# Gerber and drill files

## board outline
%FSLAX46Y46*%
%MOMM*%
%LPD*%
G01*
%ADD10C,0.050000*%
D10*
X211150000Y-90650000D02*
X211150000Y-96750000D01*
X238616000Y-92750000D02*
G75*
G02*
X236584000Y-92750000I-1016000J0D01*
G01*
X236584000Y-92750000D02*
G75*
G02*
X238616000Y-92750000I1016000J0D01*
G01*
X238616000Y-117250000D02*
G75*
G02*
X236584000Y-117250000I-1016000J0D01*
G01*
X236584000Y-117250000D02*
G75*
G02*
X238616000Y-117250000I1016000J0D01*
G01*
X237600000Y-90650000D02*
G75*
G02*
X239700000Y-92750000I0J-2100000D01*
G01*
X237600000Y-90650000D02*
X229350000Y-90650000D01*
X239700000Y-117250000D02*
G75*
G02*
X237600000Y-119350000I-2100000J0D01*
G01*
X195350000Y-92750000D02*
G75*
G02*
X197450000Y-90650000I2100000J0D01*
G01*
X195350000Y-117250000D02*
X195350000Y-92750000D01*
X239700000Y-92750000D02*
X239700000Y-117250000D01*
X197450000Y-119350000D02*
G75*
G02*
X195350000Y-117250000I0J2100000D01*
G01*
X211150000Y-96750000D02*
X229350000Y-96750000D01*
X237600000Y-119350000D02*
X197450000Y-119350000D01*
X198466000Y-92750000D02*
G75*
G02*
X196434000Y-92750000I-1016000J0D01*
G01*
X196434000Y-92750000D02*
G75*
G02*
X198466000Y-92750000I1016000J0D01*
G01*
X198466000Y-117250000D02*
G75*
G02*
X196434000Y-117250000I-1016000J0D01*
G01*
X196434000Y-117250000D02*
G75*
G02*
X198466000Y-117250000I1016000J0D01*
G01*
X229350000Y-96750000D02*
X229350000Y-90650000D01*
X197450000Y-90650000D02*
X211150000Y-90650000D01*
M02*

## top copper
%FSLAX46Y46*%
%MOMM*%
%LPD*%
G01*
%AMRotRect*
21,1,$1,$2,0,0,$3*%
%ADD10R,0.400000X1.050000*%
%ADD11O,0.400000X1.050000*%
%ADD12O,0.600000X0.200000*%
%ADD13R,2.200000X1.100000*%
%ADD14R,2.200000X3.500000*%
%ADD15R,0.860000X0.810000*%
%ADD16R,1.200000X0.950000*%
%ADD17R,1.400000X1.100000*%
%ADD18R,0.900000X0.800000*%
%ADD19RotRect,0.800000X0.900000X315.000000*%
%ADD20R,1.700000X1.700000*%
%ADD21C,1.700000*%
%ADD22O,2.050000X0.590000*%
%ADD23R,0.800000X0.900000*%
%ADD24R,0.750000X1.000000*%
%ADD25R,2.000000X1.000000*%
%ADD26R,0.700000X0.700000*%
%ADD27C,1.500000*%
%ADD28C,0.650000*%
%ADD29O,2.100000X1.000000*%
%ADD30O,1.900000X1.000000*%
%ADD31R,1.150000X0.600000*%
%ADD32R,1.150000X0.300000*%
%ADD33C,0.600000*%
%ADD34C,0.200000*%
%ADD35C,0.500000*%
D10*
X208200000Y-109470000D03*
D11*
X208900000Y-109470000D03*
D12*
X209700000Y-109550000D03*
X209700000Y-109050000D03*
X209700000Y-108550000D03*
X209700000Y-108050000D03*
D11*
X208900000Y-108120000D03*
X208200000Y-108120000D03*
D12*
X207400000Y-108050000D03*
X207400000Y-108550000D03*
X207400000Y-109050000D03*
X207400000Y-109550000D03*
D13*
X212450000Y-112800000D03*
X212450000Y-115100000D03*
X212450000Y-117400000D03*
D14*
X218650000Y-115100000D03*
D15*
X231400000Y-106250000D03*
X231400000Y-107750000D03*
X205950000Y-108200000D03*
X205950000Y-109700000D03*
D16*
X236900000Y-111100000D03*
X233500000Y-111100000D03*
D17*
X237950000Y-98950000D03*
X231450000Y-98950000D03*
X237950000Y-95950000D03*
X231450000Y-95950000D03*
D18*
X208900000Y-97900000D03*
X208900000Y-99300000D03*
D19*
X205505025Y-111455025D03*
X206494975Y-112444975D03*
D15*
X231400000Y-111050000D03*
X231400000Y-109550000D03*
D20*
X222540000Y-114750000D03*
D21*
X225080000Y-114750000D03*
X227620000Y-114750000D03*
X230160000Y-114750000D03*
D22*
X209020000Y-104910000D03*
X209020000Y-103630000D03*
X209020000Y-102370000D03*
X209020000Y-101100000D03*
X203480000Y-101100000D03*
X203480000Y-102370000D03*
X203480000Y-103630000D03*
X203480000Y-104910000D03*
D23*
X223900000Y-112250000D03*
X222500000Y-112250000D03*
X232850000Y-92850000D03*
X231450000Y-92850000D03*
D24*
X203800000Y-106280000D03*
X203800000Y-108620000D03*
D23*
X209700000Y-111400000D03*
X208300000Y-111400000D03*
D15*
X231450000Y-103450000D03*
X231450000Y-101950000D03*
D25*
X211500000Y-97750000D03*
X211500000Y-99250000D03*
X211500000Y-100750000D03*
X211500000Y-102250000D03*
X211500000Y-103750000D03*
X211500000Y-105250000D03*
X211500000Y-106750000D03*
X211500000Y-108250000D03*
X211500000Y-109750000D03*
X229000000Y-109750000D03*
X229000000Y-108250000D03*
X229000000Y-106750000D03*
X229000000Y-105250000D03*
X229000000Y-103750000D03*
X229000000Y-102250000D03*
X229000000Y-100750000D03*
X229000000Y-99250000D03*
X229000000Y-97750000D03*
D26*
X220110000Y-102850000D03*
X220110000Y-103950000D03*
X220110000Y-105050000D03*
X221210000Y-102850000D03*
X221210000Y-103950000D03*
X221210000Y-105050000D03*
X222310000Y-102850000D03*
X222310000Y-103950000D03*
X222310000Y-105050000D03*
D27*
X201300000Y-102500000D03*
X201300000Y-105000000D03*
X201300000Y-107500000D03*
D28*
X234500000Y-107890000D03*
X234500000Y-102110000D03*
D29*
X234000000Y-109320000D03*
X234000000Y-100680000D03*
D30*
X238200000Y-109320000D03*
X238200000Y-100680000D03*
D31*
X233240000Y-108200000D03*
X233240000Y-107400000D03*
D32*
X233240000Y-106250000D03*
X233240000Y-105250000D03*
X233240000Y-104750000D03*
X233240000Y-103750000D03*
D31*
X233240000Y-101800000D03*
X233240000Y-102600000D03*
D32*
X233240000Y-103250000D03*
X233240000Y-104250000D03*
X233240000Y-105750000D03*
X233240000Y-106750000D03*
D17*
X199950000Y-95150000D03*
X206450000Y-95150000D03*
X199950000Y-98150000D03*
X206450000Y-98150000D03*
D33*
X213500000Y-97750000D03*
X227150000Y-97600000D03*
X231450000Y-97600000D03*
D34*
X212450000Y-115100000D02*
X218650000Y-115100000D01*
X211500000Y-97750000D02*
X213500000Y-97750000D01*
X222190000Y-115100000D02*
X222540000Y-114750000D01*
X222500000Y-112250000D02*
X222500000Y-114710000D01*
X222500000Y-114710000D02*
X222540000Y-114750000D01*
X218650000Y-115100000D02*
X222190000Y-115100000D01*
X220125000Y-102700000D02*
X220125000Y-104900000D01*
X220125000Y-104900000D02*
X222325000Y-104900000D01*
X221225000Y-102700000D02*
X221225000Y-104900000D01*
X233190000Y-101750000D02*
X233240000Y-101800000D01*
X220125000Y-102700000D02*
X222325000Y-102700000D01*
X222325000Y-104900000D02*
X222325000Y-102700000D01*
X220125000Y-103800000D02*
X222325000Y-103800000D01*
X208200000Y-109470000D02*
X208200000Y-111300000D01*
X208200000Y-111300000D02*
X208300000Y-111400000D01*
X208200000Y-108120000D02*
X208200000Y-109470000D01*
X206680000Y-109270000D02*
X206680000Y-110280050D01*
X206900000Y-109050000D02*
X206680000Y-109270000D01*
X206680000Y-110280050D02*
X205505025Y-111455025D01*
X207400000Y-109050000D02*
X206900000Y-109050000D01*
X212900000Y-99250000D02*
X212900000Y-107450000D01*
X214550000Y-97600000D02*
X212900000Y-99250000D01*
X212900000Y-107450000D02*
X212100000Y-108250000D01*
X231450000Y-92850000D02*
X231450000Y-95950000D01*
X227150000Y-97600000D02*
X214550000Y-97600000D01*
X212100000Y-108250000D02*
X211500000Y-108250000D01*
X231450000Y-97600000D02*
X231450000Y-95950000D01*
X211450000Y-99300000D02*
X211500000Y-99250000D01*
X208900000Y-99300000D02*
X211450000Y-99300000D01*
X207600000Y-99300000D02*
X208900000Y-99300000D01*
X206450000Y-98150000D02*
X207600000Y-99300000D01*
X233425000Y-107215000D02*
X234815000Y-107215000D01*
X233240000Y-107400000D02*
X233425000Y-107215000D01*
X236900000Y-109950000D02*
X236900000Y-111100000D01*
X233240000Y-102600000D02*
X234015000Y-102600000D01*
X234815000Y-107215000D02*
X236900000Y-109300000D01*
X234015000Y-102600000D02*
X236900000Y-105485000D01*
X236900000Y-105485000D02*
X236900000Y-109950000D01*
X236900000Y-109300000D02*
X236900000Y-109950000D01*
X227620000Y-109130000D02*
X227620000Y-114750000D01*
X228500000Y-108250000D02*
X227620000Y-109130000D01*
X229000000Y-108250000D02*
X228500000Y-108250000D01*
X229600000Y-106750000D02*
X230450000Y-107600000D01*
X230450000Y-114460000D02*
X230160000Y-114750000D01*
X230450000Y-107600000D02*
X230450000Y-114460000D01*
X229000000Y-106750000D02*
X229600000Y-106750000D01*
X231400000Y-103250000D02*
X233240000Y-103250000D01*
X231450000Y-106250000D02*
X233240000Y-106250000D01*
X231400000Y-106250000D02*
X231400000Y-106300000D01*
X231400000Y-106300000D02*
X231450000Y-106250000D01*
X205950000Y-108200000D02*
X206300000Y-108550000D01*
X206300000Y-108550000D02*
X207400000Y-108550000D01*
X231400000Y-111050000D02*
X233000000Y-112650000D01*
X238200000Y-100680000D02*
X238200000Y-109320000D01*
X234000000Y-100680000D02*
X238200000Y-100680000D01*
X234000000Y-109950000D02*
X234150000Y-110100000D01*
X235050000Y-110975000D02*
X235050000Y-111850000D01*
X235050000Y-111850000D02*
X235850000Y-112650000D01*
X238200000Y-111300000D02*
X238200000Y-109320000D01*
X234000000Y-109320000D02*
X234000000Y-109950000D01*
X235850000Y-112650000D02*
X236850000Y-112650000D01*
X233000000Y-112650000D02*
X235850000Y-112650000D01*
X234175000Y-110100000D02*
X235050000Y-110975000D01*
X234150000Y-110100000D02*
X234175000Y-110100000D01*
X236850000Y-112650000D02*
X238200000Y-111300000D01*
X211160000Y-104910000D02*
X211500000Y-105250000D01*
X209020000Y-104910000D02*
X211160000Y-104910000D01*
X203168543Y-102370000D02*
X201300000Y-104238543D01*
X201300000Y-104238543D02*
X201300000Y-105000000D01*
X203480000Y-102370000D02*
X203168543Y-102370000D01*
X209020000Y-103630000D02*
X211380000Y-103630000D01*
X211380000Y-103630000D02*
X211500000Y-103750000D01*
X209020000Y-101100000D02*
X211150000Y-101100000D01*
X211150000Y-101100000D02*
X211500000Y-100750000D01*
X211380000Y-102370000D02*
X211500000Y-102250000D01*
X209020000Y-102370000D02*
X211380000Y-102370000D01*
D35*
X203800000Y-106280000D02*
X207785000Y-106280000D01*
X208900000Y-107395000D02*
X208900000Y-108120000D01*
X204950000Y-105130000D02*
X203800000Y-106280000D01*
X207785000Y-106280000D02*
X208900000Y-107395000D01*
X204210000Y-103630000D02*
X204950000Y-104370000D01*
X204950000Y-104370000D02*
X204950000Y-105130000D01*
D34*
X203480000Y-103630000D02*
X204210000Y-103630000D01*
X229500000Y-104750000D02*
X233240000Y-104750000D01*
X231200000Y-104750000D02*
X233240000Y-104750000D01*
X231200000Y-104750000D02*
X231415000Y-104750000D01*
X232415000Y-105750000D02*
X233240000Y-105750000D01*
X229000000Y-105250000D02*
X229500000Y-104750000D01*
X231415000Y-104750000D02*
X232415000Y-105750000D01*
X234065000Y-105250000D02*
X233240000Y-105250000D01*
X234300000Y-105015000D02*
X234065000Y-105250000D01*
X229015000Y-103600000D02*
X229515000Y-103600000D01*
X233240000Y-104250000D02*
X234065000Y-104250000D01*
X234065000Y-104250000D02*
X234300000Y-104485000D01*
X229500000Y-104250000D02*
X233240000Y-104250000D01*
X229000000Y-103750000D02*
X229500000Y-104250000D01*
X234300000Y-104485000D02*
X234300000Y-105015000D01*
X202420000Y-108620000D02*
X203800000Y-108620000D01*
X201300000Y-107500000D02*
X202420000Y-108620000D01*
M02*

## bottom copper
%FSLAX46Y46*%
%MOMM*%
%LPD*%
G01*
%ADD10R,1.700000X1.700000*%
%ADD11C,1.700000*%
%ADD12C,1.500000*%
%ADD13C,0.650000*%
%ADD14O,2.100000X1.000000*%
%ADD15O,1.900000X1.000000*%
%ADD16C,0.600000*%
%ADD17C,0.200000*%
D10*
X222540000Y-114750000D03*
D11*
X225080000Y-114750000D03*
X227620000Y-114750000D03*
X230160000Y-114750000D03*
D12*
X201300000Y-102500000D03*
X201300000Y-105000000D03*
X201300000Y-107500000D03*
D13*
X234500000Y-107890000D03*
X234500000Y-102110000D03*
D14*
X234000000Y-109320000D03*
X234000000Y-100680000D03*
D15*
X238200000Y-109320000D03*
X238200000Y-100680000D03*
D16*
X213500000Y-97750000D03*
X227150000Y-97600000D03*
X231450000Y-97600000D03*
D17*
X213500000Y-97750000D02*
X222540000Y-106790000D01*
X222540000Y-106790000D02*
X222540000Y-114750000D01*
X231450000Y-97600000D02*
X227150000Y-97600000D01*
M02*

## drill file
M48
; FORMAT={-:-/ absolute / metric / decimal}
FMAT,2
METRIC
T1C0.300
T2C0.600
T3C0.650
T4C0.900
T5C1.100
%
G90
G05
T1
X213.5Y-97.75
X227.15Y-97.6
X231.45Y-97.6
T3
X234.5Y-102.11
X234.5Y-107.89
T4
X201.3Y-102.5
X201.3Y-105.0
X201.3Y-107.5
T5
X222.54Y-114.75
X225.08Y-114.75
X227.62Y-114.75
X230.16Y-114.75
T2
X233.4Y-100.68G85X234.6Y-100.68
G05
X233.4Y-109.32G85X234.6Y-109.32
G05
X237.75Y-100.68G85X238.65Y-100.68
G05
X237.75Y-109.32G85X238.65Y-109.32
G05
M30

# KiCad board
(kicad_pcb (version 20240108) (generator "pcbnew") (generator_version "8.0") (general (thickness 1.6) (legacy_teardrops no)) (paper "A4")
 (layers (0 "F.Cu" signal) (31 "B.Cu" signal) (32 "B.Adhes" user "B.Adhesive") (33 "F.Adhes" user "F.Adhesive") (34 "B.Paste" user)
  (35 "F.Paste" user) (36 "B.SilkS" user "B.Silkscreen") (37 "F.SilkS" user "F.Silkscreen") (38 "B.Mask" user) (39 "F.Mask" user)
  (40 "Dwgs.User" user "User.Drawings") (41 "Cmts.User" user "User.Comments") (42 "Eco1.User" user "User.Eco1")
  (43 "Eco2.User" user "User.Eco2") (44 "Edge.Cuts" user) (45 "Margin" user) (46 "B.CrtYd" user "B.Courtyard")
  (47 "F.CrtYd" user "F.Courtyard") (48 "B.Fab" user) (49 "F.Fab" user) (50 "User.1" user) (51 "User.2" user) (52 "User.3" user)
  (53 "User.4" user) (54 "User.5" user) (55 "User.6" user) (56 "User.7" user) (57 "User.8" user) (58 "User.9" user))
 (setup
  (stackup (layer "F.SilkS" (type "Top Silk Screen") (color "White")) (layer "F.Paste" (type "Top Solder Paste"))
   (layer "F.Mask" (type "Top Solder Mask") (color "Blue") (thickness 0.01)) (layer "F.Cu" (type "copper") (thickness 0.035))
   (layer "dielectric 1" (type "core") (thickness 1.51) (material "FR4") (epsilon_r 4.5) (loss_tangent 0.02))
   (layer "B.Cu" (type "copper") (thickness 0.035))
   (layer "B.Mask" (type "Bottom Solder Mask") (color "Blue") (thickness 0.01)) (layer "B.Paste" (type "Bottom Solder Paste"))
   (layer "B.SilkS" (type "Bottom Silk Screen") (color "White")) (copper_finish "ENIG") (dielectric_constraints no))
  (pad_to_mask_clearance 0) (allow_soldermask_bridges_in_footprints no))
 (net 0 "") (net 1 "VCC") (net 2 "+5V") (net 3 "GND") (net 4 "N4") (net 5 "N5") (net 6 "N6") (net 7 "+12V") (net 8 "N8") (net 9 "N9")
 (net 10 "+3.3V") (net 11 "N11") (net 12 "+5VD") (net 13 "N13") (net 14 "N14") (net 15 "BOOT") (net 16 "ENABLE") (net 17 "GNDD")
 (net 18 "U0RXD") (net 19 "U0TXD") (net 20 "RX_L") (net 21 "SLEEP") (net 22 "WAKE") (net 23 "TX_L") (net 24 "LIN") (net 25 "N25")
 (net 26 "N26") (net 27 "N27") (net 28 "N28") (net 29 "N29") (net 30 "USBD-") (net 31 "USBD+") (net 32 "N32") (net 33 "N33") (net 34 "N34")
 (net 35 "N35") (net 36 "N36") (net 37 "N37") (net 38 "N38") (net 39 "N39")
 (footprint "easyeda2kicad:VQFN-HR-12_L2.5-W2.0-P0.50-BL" (layer "F.Cu") (at 208.55 108.8)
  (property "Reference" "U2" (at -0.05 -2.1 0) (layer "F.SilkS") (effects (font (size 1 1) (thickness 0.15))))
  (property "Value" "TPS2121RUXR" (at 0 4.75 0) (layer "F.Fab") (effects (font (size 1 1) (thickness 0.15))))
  (pad "1" smd rect (at -0.35 0.67 270) (size 1.05 0.4) (layers "F.Cu" "F.Paste" "F.Mask") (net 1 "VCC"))
  (pad "2" smd oval (at 0.35 0.67 270) (size 1.05 0.4) (layers "F.Cu" "F.Paste" "F.Mask") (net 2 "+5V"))
  (pad "3" smd oval (at 1.15 0.75) (size 0.6 0.2) (layers "F.Cu" "F.Paste" "F.Mask") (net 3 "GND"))
  (pad "4" smd oval (at 1.15 0.25) (size 0.6 0.2) (layers "F.Cu" "F.Paste" "F.Mask") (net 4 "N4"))
  (pad "5" smd oval (at 1.15 -0.25) (size 0.6 0.2) (layers "F.Cu" "F.Paste" "F.Mask") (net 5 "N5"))
  (pad "6" smd oval (at 1.15 -0.75) (size 0.6 0.2) (layers "F.Cu" "F.Paste" "F.Mask") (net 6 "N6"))
  (pad "7" smd oval (at 0.35 -0.68 270) (size 1.05 0.4) (layers "F.Cu" "F.Paste" "F.Mask") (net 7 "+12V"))
  (pad "8" smd oval (at -0.35 -0.68 270) (size 1.05 0.4) (layers "F.Cu" "F.Paste" "F.Mask") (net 1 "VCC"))
  (pad "9" smd oval (at -1.15 -0.75) (size 0.6 0.2) (layers "F.Cu" "F.Paste" "F.Mask") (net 3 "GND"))
  (pad "10" smd oval (at -1.15 -0.25) (size 0.6 0.2) (layers "F.Cu" "F.Paste" "F.Mask") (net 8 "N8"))
  (pad "11" smd oval (at -1.15 0.25) (size 0.6 0.2) (layers "F.Cu" "F.Paste" "F.Mask") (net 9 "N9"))
  (pad "12" smd oval (at -1.15 0.75) (size 0.6 0.2) (layers "F.Cu" "F.Paste" "F.Mask") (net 3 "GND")))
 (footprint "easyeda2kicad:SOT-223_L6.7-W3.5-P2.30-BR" (layer "F.Cu") (at 215.55 115.1 180)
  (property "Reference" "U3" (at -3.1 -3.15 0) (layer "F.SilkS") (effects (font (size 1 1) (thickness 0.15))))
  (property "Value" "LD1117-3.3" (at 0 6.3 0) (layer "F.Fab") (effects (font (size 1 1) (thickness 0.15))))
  (pad "1" smd rect (at 3.1 2.3 270) (size 1.1 2.2) (layers "F.Cu" "F.Paste" "F.Mask") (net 3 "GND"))
  (pad "2" smd rect (at 3.1 0 270) (size 1.1 2.2) (layers "F.Cu" "F.Paste" "F.Mask") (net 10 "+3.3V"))
  (pad "3" smd rect (at 3.1 -2.3 270) (size 1.1 2.2) (layers "F.Cu" "F.Paste" "F.Mask") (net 1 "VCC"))
  (pad "4" smd rect (at -3.1 0 180) (size 2.2 3.5) (layers "F.Cu" "F.Paste" "F.Mask") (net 10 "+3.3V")))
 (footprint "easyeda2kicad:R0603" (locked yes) (layer "F.Cu") (at 231.4 107 -90)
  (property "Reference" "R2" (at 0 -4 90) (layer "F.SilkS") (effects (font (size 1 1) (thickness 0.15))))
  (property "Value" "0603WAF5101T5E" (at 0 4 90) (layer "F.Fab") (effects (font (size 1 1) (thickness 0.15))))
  (pad "1" smd rect (at -0.75 0 270) (size 0.81 0.86) (layers "F.Cu" "F.Paste" "F.Mask") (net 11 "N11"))
  (pad "2" smd rect (at 0.75 0 270) (size 0.81 0.86) (layers "F.Cu" "F.Paste" "F.Mask") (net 3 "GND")))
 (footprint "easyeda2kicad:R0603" (layer "F.Cu") (at 205.95 108.95 -90)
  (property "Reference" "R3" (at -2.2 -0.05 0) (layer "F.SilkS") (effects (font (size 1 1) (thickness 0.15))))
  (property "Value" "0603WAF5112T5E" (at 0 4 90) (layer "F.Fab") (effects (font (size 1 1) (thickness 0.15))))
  (pad "1" smd rect (at -0.75 0 270) (size 0.81 0.86) (layers "F.Cu" "F.Paste" "F.Mask") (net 8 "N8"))
  (pad "2" smd rect (at 0.75 0 270) (size 0.81 0.86) (layers "F.Cu" "F.Paste" "F.Mask") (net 3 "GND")))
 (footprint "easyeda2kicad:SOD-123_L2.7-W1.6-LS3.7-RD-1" (layer "F.Cu") (at 235.2 111.1 180)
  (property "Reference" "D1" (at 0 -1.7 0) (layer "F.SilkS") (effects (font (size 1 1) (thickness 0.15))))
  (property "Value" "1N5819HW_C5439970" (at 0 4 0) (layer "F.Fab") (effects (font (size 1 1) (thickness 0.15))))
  (pad "1" smd rect (at -1.7 0 180) (size 1.2 0.95) (layers "F.Cu" "F.Paste" "F.Mask") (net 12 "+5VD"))
  (pad "2" smd rect (at 1.7 0 180) (size 1.2 0.95) (layers "F.Cu" "F.Paste" "F.Mask") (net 2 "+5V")))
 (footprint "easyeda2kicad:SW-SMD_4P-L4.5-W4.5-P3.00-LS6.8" (layer "F.Cu") (at 234.7 97.45 180)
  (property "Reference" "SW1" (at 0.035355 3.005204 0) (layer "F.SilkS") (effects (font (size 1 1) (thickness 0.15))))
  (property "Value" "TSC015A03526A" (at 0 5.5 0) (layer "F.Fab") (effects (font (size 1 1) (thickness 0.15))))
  (pad "1" smd rect (at -3.25 -1.5 180) (size 1.4 1.1) (layers "F.Cu" "F.Paste" "F.Mask") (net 3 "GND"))
  (pad "2" smd rect (at 3.25 -1.5 180) (size 1.4 1.1) (layers "F.Cu" "F.Paste" "F.Mask") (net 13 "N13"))
  (pad "3" smd rect (at -3.25 1.5 180) (size 1.4 1.1) (layers "F.Cu" "F.Paste" "F.Mask") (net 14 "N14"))
  (pad "4" smd rect (at 3.25 1.5 180) (size 1.4 1.1) (layers "F.Cu" "F.Paste" "F.Mask") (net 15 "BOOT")))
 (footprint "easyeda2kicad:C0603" (layer "F.Cu") (at 208.9 98.6 -90)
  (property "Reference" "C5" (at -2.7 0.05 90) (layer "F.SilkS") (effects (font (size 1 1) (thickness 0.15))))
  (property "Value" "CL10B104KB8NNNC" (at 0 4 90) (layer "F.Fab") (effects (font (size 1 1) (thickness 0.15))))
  (pad "1" smd rect (at -0.7 0 270) (size 0.8 0.9) (layers "F.Cu" "F.Paste" "F.Mask") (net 3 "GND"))
  (pad "2" smd rect (at 0.7 0 270) (size 0.8 0.9) (layers "F.Cu" "F.Paste" "F.Mask") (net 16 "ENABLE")))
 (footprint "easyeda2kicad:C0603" (layer "F.Cu") (at 206 111.95 -45)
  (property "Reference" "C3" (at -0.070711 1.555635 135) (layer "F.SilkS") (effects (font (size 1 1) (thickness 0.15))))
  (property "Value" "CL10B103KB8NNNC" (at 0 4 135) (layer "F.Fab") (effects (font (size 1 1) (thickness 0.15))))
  (pad "1" smd rect (at -0.7 0 315) (size 0.8 0.9) (layers "F.Cu" "F.Paste" "F.Mask") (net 9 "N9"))
  (pad "2" smd rect (at 0.7 0 315) (size 0.8 0.9) (layers "F.Cu" "F.Paste" "F.Mask") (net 3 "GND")))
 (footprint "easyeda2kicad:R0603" (layer "F.Cu") (at 231.4 110.3 90)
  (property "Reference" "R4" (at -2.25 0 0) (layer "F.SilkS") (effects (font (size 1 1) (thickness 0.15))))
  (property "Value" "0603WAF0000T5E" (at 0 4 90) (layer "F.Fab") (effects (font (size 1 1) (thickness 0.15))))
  (pad "1" smd rect (at -0.75 0 90) (size 0.81 0.86) (layers "F.Cu" "F.Paste" "F.Mask") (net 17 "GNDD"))
  (pad "2" smd rect (at 0.75 0 90) (size 0.81 0.86) (layers "F.Cu" "F.Paste" "F.Mask") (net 3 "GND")))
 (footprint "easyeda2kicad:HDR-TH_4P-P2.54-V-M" (layer "F.Cu") (at 226.35 114.75)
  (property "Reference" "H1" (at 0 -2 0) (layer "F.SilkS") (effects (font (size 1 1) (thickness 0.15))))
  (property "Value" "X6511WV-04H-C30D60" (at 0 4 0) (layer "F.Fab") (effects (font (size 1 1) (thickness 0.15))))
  (pad "1" thru_hole rect (at -3.81 0) (size 1.7 1.7) (drill 1.100023) (layers "*.Cu" "*.Mask") (remove_unused_layers no) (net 10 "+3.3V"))
  (pad "2" thru_hole circle (at -1.27 0) (size 1.7 1.7) (drill 1.100023) (layers "*.Cu" "*.Mask") (remove_unused_layers no) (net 3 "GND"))
  (pad "3" thru_hole circle (at 1.27 0) (size 1.7 1.7) (drill 1.100023) (layers "*.Cu" "*.Mask") (remove_unused_layers no) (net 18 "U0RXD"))
  (pad "4" thru_hole circle (at 3.81 0) (size 1.7 1.7) (drill 1.100023) (layers "*.Cu" "*.Mask") (remove_unused_layers no) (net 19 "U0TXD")))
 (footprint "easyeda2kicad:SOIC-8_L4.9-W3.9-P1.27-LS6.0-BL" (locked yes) (layer "F.Cu") (at 206.25 103 90)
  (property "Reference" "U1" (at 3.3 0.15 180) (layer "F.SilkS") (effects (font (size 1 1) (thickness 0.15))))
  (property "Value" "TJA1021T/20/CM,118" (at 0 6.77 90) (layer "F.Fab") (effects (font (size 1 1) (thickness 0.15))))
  (pad "1" smd oval (at -1.91 2.77 90) (size 0.59 2.05) (layers "F.Cu" "F.Paste" "F.Mask") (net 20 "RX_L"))
  (pad "2" smd oval (at -0.63 2.77 90) (size 0.59 2.05) (layers "F.Cu" "F.Paste" "F.Mask") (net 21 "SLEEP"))
  (pad "3" smd oval (at 0.63 2.77 90) (size 0.59 2.05) (layers "F.Cu" "F.Paste" "F.Mask") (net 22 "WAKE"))
  (pad "4" smd oval (at 1.9 2.77 90) (size 0.59 2.05) (layers "F.Cu" "F.Paste" "F.Mask") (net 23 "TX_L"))
  (pad "5" smd oval (at 1.9 -2.77 90) (size 0.59 2.05) (layers "F.Cu" "F.Paste" "F.Mask") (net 3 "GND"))
  (pad "6" smd oval (at 0.63 -2.77 90) (size 0.59 2.05) (layers "F.Cu" "F.Paste" "F.Mask") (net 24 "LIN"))
  (pad "7" smd oval (at -0.63 -2.77 90) (size 0.59 2.05) (layers "F.Cu" "F.Paste" "F.Mask") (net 7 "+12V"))
  (pad "8" smd oval (at -1.91 -2.77 90) (size 0.59 2.05) (layers "F.Cu" "F.Paste" "F.Mask") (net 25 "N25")))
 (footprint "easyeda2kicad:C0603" (layer "F.Cu") (at 223.2 112.25 180)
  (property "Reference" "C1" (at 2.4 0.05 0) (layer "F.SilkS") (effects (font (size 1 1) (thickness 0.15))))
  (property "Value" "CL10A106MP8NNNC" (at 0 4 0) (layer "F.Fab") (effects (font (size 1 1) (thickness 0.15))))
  (pad "1" smd rect (at -0.7 0 180) (size 0.8 0.9) (layers "F.Cu" "F.Paste" "F.Mask") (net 3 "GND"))
  (pad "2" smd rect (at 0.7 0 180) (size 0.8 0.9) (layers "F.Cu" "F.Paste" "F.Mask") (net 10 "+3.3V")))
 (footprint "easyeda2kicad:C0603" (layer "F.Cu") (at 232.15 92.85 180)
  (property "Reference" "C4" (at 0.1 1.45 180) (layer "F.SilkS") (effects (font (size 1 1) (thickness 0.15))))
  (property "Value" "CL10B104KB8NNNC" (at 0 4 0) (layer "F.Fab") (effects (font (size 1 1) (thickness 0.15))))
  (pad "1" smd rect (at -0.7 0 180) (size 0.8 0.9) (layers "F.Cu" "F.Paste" "F.Mask") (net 3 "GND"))
  (pad "2" smd rect (at 0.7 0 180) (size 0.8 0.9) (layers "F.Cu" "F.Paste" "F.Mask") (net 15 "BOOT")))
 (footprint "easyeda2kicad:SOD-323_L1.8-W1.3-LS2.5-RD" (layer "F.Cu") (at 203.8 107.45 -90)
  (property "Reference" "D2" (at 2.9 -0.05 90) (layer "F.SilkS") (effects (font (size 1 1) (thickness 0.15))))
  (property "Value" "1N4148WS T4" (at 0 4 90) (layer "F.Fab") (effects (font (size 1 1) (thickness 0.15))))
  (pad "1" smd rect (at -1.17 0 270) (size 1 0.75) (layers "F.Cu" "F.Paste" "F.Mask") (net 7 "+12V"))
  (pad "2" smd rect (at 1.17 0 270) (size 1 0.75) (layers "F.Cu" "F.Paste" "F.Mask") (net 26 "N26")))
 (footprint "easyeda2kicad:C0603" (layer "F.Cu") (at 209 111.4 180)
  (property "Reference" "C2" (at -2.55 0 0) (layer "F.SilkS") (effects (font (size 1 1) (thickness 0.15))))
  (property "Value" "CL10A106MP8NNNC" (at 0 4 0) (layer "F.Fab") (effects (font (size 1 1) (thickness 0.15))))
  (pad "1" smd rect (at -0.7 0 180) (size 0.8 0.9) (layers "F.Cu" "F.Paste" "F.Mask") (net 3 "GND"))
  (pad "2" smd rect (at 0.7 0 180) (size 0.8 0.9) (layers "F.Cu" "F.Paste" "F.Mask") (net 1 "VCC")))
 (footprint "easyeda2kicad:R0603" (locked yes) (layer "F.Cu") (at 231.45 102.7 90)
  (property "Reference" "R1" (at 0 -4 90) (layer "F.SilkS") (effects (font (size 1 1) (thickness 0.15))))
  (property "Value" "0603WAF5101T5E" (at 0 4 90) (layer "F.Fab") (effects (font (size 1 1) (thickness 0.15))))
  (pad "1" smd rect (at -0.75 0 90) (size 0.81 0.86) (layers "F.Cu" "F.Paste" "F.Mask") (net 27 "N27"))
  (pad "2" smd rect (at 0.75 0 90) (size 0.81 0.86) (layers "F.Cu" "F.Paste" "F.Mask") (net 3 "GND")))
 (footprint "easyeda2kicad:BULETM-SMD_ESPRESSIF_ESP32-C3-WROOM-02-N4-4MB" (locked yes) (layer "F.Cu") (at 220.25 103.75)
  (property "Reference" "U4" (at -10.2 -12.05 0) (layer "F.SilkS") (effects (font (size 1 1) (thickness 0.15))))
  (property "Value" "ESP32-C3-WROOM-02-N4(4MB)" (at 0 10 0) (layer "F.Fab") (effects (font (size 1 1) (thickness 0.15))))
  (pad "1" smd rect (at -8.75 -6) (size 2 1) (layers "F.Cu" "F.Paste" "F.Mask") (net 10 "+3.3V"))
  (pad "2" smd rect (at -8.75 -4.5) (size 2 1) (layers "F.Cu" "F.Paste" "F.Mask") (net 16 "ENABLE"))
  (pad "3" smd rect (at -8.75 -3) (size 2 1) (layers "F.Cu" "F.Paste" "F.Mask") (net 23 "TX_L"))
  (pad "4" smd rect (at -8.75 -1.5) (size 2 1) (layers "F.Cu" "F.Paste" "F.Mask") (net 22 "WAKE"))
  (pad "5" smd rect (at -8.75 0) (size 2 1) (layers "F.Cu" "F.Paste" "F.Mask") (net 21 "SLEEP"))
  (pad "6" smd rect (at -8.75 1.5) (size 2 1) (layers "F.Cu" "F.Paste" "F.Mask") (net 20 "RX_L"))
  (pad "7" smd rect (at -8.75 3) (size 2 1) (layers "F.Cu" "F.Paste" "F.Mask") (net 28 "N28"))
  (pad "8" smd rect (at -8.75 4.5) (size 2 1) (layers "F.Cu" "F.Paste" "F.Mask") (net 15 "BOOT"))
  (pad "9" smd rect (at -8.75 6) (size 2 1) (layers "F.Cu" "F.Paste" "F.Mask") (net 3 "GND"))
  (pad "10" smd rect (at 8.75 6) (size 2 1) (layers "F.Cu" "F.Paste" "F.Mask") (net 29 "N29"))
  (pad "11" smd rect (at 8.75 4.5) (size 2 1) (layers "F.Cu" "F.Paste" "F.Mask") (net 18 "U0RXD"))
  (pad "12" smd rect (at 8.75 3) (size 2 1) (layers "F.Cu" "F.Paste" "F.Mask") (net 19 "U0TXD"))
  (pad "13" smd rect (at 8.75 1.5) (size 2 1) (layers "F.Cu" "F.Paste" "F.Mask") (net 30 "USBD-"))
  (pad "14" smd rect (at 8.75 0) (size 2 1) (layers "F.Cu" "F.Paste" "F.Mask") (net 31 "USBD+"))
  (pad "15" smd rect (at 8.75 -1.5) (size 2 1) (layers "F.Cu" "F.Paste" "F.Mask") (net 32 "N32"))
  (pad "16" smd rect (at 8.75 -3) (size 2 1) (layers "F.Cu" "F.Paste" "F.Mask") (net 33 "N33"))
  (pad "17" smd rect (at 8.75 -4.5) (size 2 1) (layers "F.Cu" "F.Paste" "F.Mask") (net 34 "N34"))
  (pad "18" smd rect (at 8.75 -6) (size 2 1) (layers "F.Cu" "F.Paste" "F.Mask") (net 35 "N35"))
  (pad "19" smd rect (at -0.14 -0.9) (size 0.7 0.7) (layers "F.Cu" "F.Paste" "F.Mask") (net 3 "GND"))
  (pad "19" smd rect (at -0.14 0.2) (size 0.7 0.7) (layers "F.Cu" "F.Paste" "F.Mask") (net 3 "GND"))
  (pad "19" smd rect (at -0.14 1.3) (size 0.7 0.7) (layers "F.Cu" "F.Paste" "F.Mask") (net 3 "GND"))
  (pad "19" smd rect (at 0.96 -0.9) (size 0.7 0.7) (layers "F.Cu" "F.Paste" "F.Mask") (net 3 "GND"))
  (pad "19" smd rect (at 0.96 0.2) (size 0.7 0.7) (layers "F.Cu" "F.Paste" "F.Mask") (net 3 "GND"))
  (pad "19" smd rect (at 0.96 1.3) (size 0.7 0.7) (layers "F.Cu" "F.Paste" "F.Mask") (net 3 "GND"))
  (pad "19" smd rect (at 2.06 -0.9) (size 0.7 0.7) (layers "F.Cu" "F.Paste" "F.Mask") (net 3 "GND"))
  (pad "19" smd rect (at 2.06 0.2) (size 0.7 0.7) (layers "F.Cu" "F.Paste" "F.Mask") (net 3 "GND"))
  (pad "19" smd rect (at 2.06 1.3) (size 0.7 0.7) (layers "F.Cu" "F.Paste" "F.Mask") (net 3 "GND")))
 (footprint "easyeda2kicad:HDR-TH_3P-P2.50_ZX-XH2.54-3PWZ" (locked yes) (layer "F.Cu") (at 201.3 105 -90)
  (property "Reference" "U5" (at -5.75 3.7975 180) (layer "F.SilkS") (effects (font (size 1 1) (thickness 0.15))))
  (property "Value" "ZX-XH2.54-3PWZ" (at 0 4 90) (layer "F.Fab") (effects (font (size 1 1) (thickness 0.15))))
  (pad "1" thru_hole circle (at -2.5 0 270) (size 1.5 1.5) (drill 0.900024) (layers "*.Cu" "*.Mask") (remove_unused_layers no) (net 3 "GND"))
  (pad "2" thru_hole circle (at 0 0 270) (size 1.5 1.5) (drill 0.900024) (layers "*.Cu" "*.Mask") (remove_unused_layers no) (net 24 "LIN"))
  (pad "3" thru_hole circle (at 2.5 0 270) (size 1.5 1.5) (drill 0.900024) (layers "*.Cu" "*.Mask") (remove_unused_layers no) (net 26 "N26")))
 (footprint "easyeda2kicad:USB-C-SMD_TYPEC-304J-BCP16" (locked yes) (layer "F.Cu") (at 235.72 105 90)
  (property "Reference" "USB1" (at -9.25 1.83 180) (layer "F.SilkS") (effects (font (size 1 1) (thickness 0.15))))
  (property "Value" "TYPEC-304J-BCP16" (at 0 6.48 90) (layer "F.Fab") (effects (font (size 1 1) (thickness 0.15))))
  (pad "" thru_hole circle (at -2.89 -1.22 90) (size 0.65 0.65) (drill 0.65) (layers "*.Cu" "*.Mask") (remove_unused_layers no))
  (pad "" thru_hole circle (at 2.89 -1.22 90) (size 0.65 0.65) (drill 0.65) (layers "*.Cu" "*.Mask") (remove_unused_layers no))
  (pad "13" thru_hole oval (at -4.32 -1.72 90) (size 1 2.1) (drill oval 0.599999 1.799996) (layers "*.Cu" "*.Mask")
   (remove_unused_layers no) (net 17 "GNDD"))
  (pad "14" thru_hole oval (at 4.32 -1.72 90) (size 1 2.1) (drill oval 0.599999 1.799996) (layers "*.Cu" "*.Mask") (remove_unused_layers no)
   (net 17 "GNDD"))
  (pad "15" thru_hole oval (at -4.32 2.48 90) (size 1 1.9) (drill oval 0.599999 1.500022) (layers "*.Cu" "*.Mask") (remove_unused_layers no)
   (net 17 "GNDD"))
  (pad "16" thru_hole oval (at 4.32 2.48 90) (size 1 1.9) (drill oval 0.599999 1.500022) (layers "*.Cu" "*.Mask") (remove_unused_layers no)
   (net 17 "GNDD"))
  (pad "A1B12" smd rect (at -3.2 -2.48 90) (size 0.6 1.15) (layers "F.Cu" "F.Paste" "F.Mask") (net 3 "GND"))
  (pad "A4B9" smd rect (at -2.4 -2.48 90) (size 0.6 1.15) (layers "F.Cu" "F.Paste" "F.Mask") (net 12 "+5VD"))
  (pad "A5" smd rect (at -1.25 -2.48 90) (size 0.3 1.15) (layers "F.Cu" "F.Paste" "F.Mask") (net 11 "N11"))
  (pad "A6" smd rect (at -0.25 -2.48 90) (size 0.3 1.15) (layers "F.Cu" "F.Paste" "F.Mask") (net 31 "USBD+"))
  (pad "A7" smd rect (at 0.25 -2.48 90) (size 0.3 1.15) (layers "F.Cu" "F.Paste" "F.Mask") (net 30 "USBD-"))
  (pad "A8" smd rect (at 1.25 -2.48 90) (size 0.3 1.15) (layers "F.Cu" "F.Paste" "F.Mask") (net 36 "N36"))
  (pad "B1A12" smd rect (at 3.2 -2.48 90) (size 0.6 1.15) (layers "F.Cu" "F.Paste" "F.Mask") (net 3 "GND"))
  (pad "B4A9" smd rect (at 2.4 -2.48 90) (size 0.6 1.15) (layers "F.Cu" "F.Paste" "F.Mask") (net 12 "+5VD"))
  (pad "B5" smd rect (at 1.75 -2.48 90) (size 0.3 1.15) (layers "F.Cu" "F.Paste" "F.Mask") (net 27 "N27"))
  (pad "B6" smd rect (at 0.75 -2.48 90) (size 0.3 1.15) (layers "F.Cu" "F.Paste" "F.Mask") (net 31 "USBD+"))
  (pad "B7" smd rect (at -0.75 -2.48 90) (size 0.3 1.15) (layers "F.Cu" "F.Paste" "F.Mask") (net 30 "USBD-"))
  (pad "B8" smd rect (at -1.75 -2.48 90) (size 0.3 1.15) (layers "F.Cu" "F.Paste" "F.Mask") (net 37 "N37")))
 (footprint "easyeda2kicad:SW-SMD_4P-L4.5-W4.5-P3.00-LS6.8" (layer "F.Cu") (at 203.2 96.65)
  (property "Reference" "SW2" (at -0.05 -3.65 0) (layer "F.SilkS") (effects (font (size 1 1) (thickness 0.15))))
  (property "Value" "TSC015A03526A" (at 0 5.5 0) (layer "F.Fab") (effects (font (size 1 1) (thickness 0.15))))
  (pad "1" smd rect (at -3.25 -1.5) (size 1.4 1.1) (layers "F.Cu" "F.Paste" "F.Mask") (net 3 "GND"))
  (pad "2" smd rect (at 3.25 -1.5) (size 1.4 1.1) (layers "F.Cu" "F.Paste" "F.Mask") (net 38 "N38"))
  (pad "3" smd rect (at -3.25 1.5) (size 1.4 1.1) (layers "F.Cu" "F.Paste" "F.Mask") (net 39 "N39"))
  (pad "4" smd rect (at 3.25 1.5) (size 1.4 1.1) (layers "F.Cu" "F.Paste" "F.Mask") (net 16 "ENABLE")))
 (gr_line (start 211.15 90.65) (end 211.15 96.75) (stroke (width 0.05) (type default)) (layer "Edge.Cuts"))
 (gr_circle (center 237.6 92.75) (end 238.616 92.75) (stroke (width 0.05) (type default)) (fill none) (layer "Edge.Cuts"))
 (gr_circle (center 237.6 117.25) (end 238.616 117.25) (stroke (width 0.05) (type default)) (fill none) (layer "Edge.Cuts"))
 (gr_arc (start 237.6 90.65) (mid 239.084924 91.265076) (end 239.7 92.75) (stroke (width 0.05) (type default)) (layer "Edge.Cuts"))
 (gr_line (start 237.6 90.65) (end 229.35 90.65) (stroke (width 0.05) (type default)) (layer "Edge.Cuts"))
 (gr_arc (start 239.7 117.25) (mid 239.084924 118.734924) (end 237.6 119.35) (stroke (width 0.05) (type default)) (layer "Edge.Cuts"))
 (gr_arc (start 195.35 92.75) (mid 195.965076 91.265076) (end 197.45 90.65) (stroke (width 0.05) (type default)) (layer "Edge.Cuts"))
 (gr_line (start 195.35 117.25) (end 195.35 92.75) (stroke (width 0.05) (type default)) (layer "Edge.Cuts"))
 (gr_line (start 239.7 92.75) (end 239.7 117.25) (stroke (width 0.05) (type default)) (layer "Edge.Cuts"))
 (gr_arc (start 197.45 119.35) (mid 195.965076 118.734924) (end 195.35 117.25) (stroke (width 0.05) (type default)) (layer "Edge.Cuts"))
 (gr_line (start 211.15 96.75) (end 229.35 96.75) (stroke (width 0.05) (type default)) (layer "Edge.Cuts"))
 (gr_line (start 237.6 119.35) (end 197.45 119.35) (stroke (width 0.05) (type default)) (layer "Edge.Cuts"))
 (gr_circle (center 197.45 92.75) (end 198.466 92.75) (stroke (width 0.05) (type default)) (fill none) (layer "Edge.Cuts"))
 (gr_circle (center 197.45 117.25) (end 198.466 117.25) (stroke (width 0.05) (type default)) (fill none) (layer "Edge.Cuts"))
 (gr_line (start 229.35 96.75) (end 229.35 90.65) (stroke (width 0.05) (type default)) (layer "Edge.Cuts"))
 (gr_line (start 197.45 90.65) (end 211.15 90.65) (stroke (width 0.05) (type default)) (layer "Edge.Cuts"))
 (segment (start 212.45 115.1) (end 218.65 115.1) (width 0.2) (layer "F.Cu") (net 10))
 (segment (start 211.5 97.75) (end 213.5 97.75) (width 0.2) (layer "F.Cu") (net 10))
 (segment (start 222.19 115.1) (end 222.54 114.75) (width 0.2) (layer "F.Cu") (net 10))
 (segment (start 222.5 112.25) (end 222.5 114.71) (width 0.2) (layer "F.Cu") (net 10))
 (segment (start 222.5 114.71) (end 222.54 114.75) (width 0.2) (layer "F.Cu") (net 10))
 (segment (start 218.65 115.1) (end 222.19 115.1) (width 0.2) (layer "F.Cu") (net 10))
 (via (at 213.5 97.75) (size 0.6) (drill 0.3) (layers "F.Cu" "B.Cu") (free yes) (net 10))
 (segment (start 213.5 97.75) (end 222.54 106.79) (width 0.2) (layer "B.Cu") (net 10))
 (segment (start 222.54 106.79) (end 222.54 114.75) (width 0.2) (layer "B.Cu") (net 10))
 (segment (start 220.125 102.7) (end 220.125 104.9) (width 0.2) (layer "F.Cu") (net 3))
 (segment (start 220.125 104.9) (end 222.325 104.9) (width 0.2) (layer "F.Cu") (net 3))
 (segment (start 221.225 102.7) (end 221.225 104.9) (width 0.2) (layer "F.Cu") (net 3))
 (segment (start 233.19 101.75) (end 233.24 101.8) (width 0.2) (layer "F.Cu") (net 3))
 (segment (start 220.125 102.7) (end 222.325 102.7) (width 0.2) (layer "F.Cu") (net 3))
 (segment (start 222.325 104.9) (end 222.325 102.7) (width 0.2) (layer "F.Cu") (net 3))
 (segment (start 220.125 103.8) (end 222.325 103.8) (width 0.2) (layer "F.Cu") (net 3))
 (segment (start 208.2 109.47) (end 208.2 111.3) (width 0.2) (layer "F.Cu") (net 1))
 (segment (start 208.2 111.3) (end 208.3 111.4) (width 0.2) (layer "F.Cu") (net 1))
 (segment (start 208.2 108.12) (end 208.2 109.47) (width 0.2) (layer "F.Cu") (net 1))
 (segment (start 206.68 109.27) (end 206.68 110.28005) (width 0.2) (layer "F.Cu") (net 9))
 (segment (start 206.9 109.05) (end 206.68 109.27) (width 0.2) (layer "F.Cu") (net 9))
 (segment (start 206.68 110.28005) (end 205.505025 111.455025) (width 0.2) (layer "F.Cu") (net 9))
 (segment (start 207.4 109.05) (end 206.9 109.05) (width 0.2) (layer "F.Cu") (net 9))
 (segment (start 212.9 99.25) (end 212.9 107.45) (width 0.2) (layer "F.Cu") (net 15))
 (segment (start 214.55 97.6) (end 212.9 99.25) (width 0.2) (layer "F.Cu") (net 15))
 (segment (start 212.9 107.45) (end 212.1 108.25) (width 0.2) (layer "F.Cu") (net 15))
 (segment (start 231.45 92.85) (end 231.45 95.95) (width 0.2) (layer "F.Cu") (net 15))
 (segment (start 227.15 97.6) (end 214.55 97.6) (width 0.2) (layer "F.Cu") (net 15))
 (segment (start 212.1 108.25) (end 211.5 108.25) (width 0.2) (layer "F.Cu") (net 15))
 (segment (start 231.45 97.6) (end 231.45 95.95) (width 0.2) (layer "F.Cu") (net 15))
 (via (at 227.15 97.6) (size 0.6) (drill 0.3) (layers "F.Cu" "B.Cu") (free yes) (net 15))
 (via (at 231.45 97.6) (size 0.6) (drill 0.3) (layers "F.Cu" "B.Cu") (free yes) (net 15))
 (segment (start 231.45 97.6) (end 227.15 97.6) (width 0.2) (layer "B.Cu") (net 15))
 (segment (start 211.45 99.3) (end 211.5 99.25) (width 0.2) (layer "F.Cu") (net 16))
 (segment (start 208.9 99.3) (end 211.45 99.3) (width 0.2) (layer "F.Cu") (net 16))
 (segment (start 207.6 99.3) (end 208.9 99.3) (width 0.2) (layer "F.Cu") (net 16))
 (segment (start 206.45 98.15) (end 207.6 99.3) (width 0.2) (layer "F.Cu") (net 16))
 (segment (start 233.425 107.215) (end 234.815 107.215) (width 0.2) (layer "F.Cu") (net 12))
 (segment (start 233.24 107.4) (end 233.425 107.215) (width 0.2) (layer "F.Cu") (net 12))
 (segment (start 236.9 109.95) (end 236.9 111.1) (width 0.2) (layer "F.Cu") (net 12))
 (segment (start 233.24 102.6) (end 234.015 102.6) (width 0.2) (layer "F.Cu") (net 12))
 (segment (start 234.815 107.215) (end 236.9 109.3) (width 0.2) (layer "F.Cu") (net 12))
 (segment (start 234.015 102.6) (end 236.9 105.485) (width 0.2) (layer "F.Cu") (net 12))
 (segment (start 236.9 105.485) (end 236.9 109.95) (width 0.2) (layer "F.Cu") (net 12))
 (segment (start 236.9 109.3) (end 236.9 109.95) (width 0.2) (layer "F.Cu") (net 12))
 (segment (start 227.62 109.13) (end 227.62 114.75) (width 0.2) (layer "F.Cu") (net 18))
 (segment (start 228.5 108.25) (end 227.62 109.13) (width 0.2) (layer "F.Cu") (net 18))
 (segment (start 229 108.25) (end 228.5 108.25) (width 0.2) (layer "F.Cu") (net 18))
 (segment (start 229.6 106.75) (end 230.45 107.6) (width 0.2) (layer "F.Cu") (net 19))
 (segment (start 230.45 114.46) (end 230.16 114.75) (width 0.2) (layer "F.Cu") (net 19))
 (segment (start 230.45 107.6) (end 230.45 114.46) (width 0.2) (layer "F.Cu") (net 19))
 (segment (start 229 106.75) (end 229.6 106.75) (width 0.2) (layer "F.Cu") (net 19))
 (segment (start 231.4 103.25) (end 233.24 103.25) (width 0.2) (layer "F.Cu") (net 27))
 (segment (start 231.45 106.25) (end 233.24 106.25) (width 0.2) (layer "F.Cu") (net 11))
 (segment (start 231.4 106.25) (end 231.4 106.3) (width 0.2) (layer "F.Cu") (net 11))
 (segment (start 231.4 106.3) (end 231.45 106.25) (width 0.2) (layer "F.Cu") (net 11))
 (segment (start 205.95 108.2) (end 206.3 108.55) (width 0.2) (layer "F.Cu") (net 8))
 (segment (start 206.3 108.55) (end 207.4 108.55) (width 0.2) (layer "F.Cu") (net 8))
 (segment (start 231.4 111.05) (end 233 112.65) (width 0.2) (layer "F.Cu") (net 17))
 (segment (start 238.2 100.68) (end 238.2 109.32) (width 0.2) (layer "F.Cu") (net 17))
 (segment (start 234 100.68) (end 238.2 100.68) (width 0.2) (layer "F.Cu") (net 17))
 (segment (start 234 109.95) (end 234.15 110.1) (width 0.2) (layer "F.Cu") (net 17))
 (segment (start 235.05 110.975) (end 235.05 111.85) (width 0.2) (layer "F.Cu") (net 17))
 (segment (start 235.05 111.85) (end 235.85 112.65) (width 0.2) (layer "F.Cu") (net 17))
 (segment (start 238.2 111.3) (end 238.2 109.32) (width 0.2) (layer "F.Cu") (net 17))
 (segment (start 234 109.32) (end 234 109.95) (width 0.2) (layer "F.Cu") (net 17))
 (segment (start 235.85 112.65) (end 236.85 112.65) (width 0.2) (layer "F.Cu") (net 17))
 (segment (start 233 112.65) (end 235.85 112.65) (width 0.2) (layer "F.Cu") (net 17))
 (segment (start 234.175 110.1) (end 235.05 110.975) (width 0.2) (layer "F.Cu") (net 17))
 (segment (start 234.15 110.1) (end 234.175 110.1) (width 0.2) (layer "F.Cu") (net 17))
 (segment (start 236.85 112.65) (end 238.2 111.3) (width 0.2) (layer "F.Cu") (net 17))
 (segment (start 211.16 104.91) (end 211.5 105.25) (width 0.2) (layer "F.Cu") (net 20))
 (segment (start 209.02 104.91) (end 211.16 104.91) (width 0.2) (layer "F.Cu") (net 20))
 (segment (start 203.168543 102.37) (end 201.3 104.238543) (width 0.2) (layer "F.Cu") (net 24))
 (segment (start 201.3 104.238543) (end 201.3 105) (width 0.2) (layer "F.Cu") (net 24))
 (segment (start 203.48 102.37) (end 203.168543 102.37) (width 0.2) (layer "F.Cu") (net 24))
 (segment (start 209.02 103.63) (end 211.38 103.63) (width 0.2) (layer "F.Cu") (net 21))
 (segment (start 211.38 103.63) (end 211.5 103.75) (width 0.2) (layer "F.Cu") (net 21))
 (segment (start 209.02 101.1) (end 211.15 101.1) (width 0.2) (layer "F.Cu") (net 23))
 (segment (start 211.15 101.1) (end 211.5 100.75) (width 0.2) (layer "F.Cu") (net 23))
 (segment (start 211.38 102.37) (end 211.5 102.25) (width 0.2) (layer "F.Cu") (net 22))
 (segment (start 209.02 102.37) (end 211.38 102.37) (width 0.2) (layer "F.Cu") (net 22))
 (segment (start 203.8 106.28) (end 207.785 106.28) (width 0.5) (layer "F.Cu") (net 7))
 (segment (start 208.9 107.395) (end 208.9 108.12) (width 0.5) (layer "F.Cu") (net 7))
 (segment (start 204.95 105.13) (end 203.8 106.28) (width 0.5) (layer "F.Cu") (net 7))
 (segment (start 207.785 106.28) (end 208.9 107.395) (width 0.5) (layer "F.Cu") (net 7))
 (segment (start 204.21 103.63) (end 204.95 104.37) (width 0.5) (layer "F.Cu") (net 7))
 (segment (start 204.95 104.37) (end 204.95 105.13) (width 0.5) (layer "F.Cu") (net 7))
 (segment (start 203.48 103.63) (end 204.21 103.63) (width 0.2) (layer "F.Cu") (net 7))
 (segment (start 229.5 104.75) (end 233.24 104.75) (width 0.2) (layer "F.Cu") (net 30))
 (segment (start 231.2 104.75) (end 233.24 104.75) (width 0.2) (layer "F.Cu") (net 30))
 (segment (start 231.2 104.75) (end 231.415 104.75) (width 0.2) (layer "F.Cu") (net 30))
 (segment (start 232.415 105.75) (end 233.24 105.75) (width 0.2) (layer "F.Cu") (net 30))
 (segment (start 229 105.25) (end 229.5 104.75) (width 0.2) (layer "F.Cu") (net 30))
 (segment (start 231.415 104.75) (end 232.415 105.75) (width 0.2) (layer "F.Cu") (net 30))
 (segment (start 234.065 105.25) (end 233.24 105.25) (width 0.2) (layer "F.Cu") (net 31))
 (segment (start 234.3 105.015) (end 234.065 105.25) (width 0.2) (layer "F.Cu") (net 31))
 (segment (start 229.015 103.6) (end 229.515 103.6) (width 0.2) (layer "F.Cu") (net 31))
 (segment (start 233.24 104.25) (end 234.065 104.25) (width 0.2) (layer "F.Cu") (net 31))
 (segment (start 234.065 104.25) (end 234.3 104.485) (width 0.2) (layer "F.Cu") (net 31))
 (segment (start 229.5 104.25) (end 233.24 104.25) (width 0.2) (layer "F.Cu") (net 31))
 (segment (start 229 103.75) (end 229.5 104.25) (width 0.2) (layer "F.Cu") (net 31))
 (segment (start 234.3 104.485) (end 234.3 105.015) (width 0.2) (layer "F.Cu") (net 31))
 (segment (start 202.42 108.62) (end 203.8 108.62) (width 0.2) (layer "F.Cu") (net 26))
 (segment (start 201.3 107.5) (end 202.42 108.62) (width 0.2) (layer "F.Cu") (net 26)))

